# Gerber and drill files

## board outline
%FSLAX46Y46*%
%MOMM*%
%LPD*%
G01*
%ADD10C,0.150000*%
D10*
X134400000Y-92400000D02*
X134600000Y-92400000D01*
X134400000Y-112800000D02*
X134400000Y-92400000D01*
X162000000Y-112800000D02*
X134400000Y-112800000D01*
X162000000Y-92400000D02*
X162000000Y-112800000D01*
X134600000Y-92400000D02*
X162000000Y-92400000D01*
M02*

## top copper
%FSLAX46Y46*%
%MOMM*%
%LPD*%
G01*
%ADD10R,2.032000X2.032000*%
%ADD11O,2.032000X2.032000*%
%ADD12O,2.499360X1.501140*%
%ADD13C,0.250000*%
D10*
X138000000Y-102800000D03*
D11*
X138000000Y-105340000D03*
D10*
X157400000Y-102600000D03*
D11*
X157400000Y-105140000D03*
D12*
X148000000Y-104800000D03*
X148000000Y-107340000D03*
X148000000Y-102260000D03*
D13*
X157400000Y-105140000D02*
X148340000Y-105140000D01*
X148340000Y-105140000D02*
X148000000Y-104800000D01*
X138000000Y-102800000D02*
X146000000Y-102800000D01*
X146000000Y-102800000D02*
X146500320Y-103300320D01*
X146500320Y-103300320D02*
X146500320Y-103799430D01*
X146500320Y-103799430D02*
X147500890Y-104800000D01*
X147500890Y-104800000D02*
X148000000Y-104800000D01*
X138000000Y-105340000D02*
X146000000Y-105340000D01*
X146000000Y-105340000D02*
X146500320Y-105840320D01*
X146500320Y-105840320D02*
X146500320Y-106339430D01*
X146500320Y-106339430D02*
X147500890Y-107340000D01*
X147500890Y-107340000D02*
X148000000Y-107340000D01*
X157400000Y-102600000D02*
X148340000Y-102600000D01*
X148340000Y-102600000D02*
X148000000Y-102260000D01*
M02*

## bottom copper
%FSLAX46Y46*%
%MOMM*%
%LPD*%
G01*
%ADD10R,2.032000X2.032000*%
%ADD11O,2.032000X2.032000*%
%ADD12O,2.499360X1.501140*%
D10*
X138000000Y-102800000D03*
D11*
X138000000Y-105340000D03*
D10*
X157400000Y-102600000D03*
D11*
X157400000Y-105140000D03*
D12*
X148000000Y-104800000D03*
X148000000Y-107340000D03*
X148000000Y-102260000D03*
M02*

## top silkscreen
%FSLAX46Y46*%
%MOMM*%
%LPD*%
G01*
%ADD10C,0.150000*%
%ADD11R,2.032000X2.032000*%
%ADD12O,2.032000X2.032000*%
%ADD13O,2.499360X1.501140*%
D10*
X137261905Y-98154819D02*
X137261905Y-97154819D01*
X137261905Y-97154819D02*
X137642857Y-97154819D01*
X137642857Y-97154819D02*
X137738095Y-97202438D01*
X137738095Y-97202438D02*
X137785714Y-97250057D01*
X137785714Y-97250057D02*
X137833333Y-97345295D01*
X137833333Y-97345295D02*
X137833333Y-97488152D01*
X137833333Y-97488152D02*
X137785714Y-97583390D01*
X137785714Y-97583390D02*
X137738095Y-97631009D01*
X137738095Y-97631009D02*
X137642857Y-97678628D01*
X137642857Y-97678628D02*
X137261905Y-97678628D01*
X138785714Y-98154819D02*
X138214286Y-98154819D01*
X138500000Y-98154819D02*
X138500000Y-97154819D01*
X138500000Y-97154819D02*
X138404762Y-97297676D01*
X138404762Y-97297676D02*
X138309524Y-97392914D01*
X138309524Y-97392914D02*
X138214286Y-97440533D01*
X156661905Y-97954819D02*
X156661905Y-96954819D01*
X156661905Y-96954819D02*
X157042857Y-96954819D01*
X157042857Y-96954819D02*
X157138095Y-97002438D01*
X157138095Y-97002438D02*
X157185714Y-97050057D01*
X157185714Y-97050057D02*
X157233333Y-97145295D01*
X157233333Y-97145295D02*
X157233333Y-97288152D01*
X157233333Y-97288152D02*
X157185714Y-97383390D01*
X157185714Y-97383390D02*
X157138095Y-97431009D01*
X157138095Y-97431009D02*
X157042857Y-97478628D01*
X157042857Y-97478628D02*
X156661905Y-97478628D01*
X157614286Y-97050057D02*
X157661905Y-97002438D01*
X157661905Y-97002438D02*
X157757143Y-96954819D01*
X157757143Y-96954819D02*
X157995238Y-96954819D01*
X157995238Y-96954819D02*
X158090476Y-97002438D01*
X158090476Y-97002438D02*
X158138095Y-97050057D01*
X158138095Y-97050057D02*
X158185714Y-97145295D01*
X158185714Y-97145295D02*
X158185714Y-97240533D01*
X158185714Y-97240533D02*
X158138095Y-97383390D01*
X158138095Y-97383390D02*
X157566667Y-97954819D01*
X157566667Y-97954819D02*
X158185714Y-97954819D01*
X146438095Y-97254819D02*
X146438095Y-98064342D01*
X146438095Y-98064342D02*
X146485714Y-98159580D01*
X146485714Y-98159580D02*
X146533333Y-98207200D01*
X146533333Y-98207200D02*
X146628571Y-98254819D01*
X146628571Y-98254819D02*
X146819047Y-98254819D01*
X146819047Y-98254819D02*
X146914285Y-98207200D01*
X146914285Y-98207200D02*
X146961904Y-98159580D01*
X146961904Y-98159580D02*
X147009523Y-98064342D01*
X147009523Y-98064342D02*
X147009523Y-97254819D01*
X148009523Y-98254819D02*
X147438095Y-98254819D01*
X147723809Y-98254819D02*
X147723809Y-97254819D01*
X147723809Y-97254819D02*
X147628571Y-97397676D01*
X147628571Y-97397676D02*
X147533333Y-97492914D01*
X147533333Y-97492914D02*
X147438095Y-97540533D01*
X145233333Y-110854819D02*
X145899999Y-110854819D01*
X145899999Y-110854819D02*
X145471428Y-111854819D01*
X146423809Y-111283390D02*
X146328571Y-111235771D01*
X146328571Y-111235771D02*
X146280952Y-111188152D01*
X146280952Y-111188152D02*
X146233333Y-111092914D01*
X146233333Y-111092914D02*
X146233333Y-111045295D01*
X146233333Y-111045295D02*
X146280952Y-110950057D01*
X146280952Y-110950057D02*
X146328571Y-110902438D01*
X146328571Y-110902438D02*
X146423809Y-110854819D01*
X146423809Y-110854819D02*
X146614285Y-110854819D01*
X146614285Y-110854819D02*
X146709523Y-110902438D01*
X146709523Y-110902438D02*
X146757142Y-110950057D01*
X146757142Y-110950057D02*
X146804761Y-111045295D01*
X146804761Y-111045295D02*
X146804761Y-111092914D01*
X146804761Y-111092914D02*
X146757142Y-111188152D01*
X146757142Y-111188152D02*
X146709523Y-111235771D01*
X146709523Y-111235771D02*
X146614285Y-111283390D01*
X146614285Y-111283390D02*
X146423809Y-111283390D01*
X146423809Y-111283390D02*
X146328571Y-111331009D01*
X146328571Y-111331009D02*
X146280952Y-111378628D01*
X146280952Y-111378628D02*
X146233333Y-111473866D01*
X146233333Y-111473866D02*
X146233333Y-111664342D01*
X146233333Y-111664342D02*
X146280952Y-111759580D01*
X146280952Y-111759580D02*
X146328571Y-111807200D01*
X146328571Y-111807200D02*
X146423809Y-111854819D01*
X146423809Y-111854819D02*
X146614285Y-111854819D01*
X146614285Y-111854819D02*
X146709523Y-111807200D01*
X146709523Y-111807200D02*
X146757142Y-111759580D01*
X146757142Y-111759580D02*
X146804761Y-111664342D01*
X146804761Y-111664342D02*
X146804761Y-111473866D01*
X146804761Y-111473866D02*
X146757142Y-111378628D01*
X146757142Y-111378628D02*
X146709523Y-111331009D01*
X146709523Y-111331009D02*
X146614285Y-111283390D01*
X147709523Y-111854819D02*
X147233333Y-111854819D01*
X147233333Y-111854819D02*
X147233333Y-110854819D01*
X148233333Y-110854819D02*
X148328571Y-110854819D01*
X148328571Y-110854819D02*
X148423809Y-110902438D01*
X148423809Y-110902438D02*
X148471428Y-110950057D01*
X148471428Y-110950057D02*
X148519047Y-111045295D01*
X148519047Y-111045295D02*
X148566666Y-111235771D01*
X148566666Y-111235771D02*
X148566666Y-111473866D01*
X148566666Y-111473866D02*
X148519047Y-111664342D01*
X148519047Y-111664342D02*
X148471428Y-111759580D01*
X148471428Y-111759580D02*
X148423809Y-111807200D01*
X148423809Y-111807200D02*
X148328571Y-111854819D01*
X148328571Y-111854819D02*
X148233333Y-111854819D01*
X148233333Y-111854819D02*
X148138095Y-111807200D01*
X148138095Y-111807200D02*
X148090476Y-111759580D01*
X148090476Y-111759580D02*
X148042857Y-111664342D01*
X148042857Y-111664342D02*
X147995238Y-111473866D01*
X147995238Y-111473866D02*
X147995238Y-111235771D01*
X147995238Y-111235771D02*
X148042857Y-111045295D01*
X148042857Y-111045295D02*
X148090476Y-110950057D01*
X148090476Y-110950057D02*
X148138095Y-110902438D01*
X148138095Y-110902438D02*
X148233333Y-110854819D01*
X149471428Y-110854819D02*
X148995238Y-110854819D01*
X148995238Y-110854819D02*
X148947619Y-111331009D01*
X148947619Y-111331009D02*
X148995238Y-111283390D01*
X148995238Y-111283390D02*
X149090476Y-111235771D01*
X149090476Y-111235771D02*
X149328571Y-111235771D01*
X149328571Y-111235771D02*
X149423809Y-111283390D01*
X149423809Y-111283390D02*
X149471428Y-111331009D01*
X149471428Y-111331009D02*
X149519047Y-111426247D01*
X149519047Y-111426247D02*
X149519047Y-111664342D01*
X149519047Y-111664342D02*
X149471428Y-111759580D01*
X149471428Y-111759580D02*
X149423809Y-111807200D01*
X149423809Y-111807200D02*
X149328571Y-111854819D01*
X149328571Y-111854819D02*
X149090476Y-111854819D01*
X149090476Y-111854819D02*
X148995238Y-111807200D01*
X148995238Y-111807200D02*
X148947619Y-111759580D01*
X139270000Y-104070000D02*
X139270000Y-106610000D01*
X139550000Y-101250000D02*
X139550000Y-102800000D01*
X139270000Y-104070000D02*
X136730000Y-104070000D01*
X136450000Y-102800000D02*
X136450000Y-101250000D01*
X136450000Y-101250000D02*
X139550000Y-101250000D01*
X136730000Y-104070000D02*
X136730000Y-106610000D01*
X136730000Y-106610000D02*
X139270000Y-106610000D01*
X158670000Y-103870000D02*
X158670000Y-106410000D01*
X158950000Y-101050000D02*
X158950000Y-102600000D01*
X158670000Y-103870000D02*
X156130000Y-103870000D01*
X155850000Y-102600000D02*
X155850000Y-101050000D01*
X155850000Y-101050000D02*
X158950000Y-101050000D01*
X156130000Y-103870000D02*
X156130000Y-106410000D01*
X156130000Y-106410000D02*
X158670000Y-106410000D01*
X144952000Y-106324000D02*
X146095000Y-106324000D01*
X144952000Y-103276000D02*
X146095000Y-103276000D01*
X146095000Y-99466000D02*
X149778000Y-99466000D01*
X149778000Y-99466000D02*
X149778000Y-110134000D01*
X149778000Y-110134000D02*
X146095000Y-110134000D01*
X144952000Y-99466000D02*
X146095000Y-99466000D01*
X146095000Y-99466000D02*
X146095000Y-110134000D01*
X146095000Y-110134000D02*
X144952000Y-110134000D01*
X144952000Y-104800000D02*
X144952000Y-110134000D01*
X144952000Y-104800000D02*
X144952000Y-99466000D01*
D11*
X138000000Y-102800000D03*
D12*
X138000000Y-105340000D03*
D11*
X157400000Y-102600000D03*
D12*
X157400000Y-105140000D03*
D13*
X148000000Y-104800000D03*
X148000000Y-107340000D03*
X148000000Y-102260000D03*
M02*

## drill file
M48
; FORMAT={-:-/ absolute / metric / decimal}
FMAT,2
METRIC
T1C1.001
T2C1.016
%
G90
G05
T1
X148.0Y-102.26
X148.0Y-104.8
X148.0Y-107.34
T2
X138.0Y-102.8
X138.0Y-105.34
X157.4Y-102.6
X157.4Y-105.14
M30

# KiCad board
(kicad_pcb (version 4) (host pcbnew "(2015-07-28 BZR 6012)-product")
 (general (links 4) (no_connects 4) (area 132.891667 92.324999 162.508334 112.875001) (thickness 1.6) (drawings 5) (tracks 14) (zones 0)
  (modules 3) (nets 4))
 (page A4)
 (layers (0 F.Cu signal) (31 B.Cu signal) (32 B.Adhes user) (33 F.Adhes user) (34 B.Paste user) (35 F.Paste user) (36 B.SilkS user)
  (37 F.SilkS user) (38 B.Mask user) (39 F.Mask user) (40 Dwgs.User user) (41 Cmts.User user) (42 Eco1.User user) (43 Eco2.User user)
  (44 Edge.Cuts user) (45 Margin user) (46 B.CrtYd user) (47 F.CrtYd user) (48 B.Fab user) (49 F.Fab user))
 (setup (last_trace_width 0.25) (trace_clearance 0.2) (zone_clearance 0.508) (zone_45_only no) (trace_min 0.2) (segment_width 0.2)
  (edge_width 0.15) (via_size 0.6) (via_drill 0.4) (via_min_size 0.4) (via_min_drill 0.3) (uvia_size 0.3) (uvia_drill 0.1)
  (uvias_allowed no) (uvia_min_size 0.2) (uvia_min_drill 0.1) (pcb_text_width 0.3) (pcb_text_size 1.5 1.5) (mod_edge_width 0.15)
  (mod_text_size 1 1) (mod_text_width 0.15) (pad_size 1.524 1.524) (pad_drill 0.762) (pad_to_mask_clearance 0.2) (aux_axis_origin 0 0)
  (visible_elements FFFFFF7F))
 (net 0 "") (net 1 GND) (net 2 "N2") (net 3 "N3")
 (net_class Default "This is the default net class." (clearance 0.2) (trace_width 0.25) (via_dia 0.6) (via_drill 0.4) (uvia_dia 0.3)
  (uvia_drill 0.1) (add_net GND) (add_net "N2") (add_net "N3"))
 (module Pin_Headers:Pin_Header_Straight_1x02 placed (layer F.Cu) (at 138 102.8)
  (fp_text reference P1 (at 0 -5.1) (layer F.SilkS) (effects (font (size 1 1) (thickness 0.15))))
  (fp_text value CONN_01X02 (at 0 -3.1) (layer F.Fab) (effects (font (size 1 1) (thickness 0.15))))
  (fp_line (start 1.27 1.27) (end 1.27 3.81) (layer F.SilkS) (width 0.15))
  (fp_line (start 1.55 -1.55) (end 1.55 0) (layer F.SilkS) (width 0.15))
  (fp_line (start 1.27 1.27) (end -1.27 1.27) (layer F.SilkS) (width 0.15))
  (fp_line (start -1.55 0) (end -1.55 -1.55) (layer F.SilkS) (width 0.15))
  (fp_line (start -1.55 -1.55) (end 1.55 -1.55) (layer F.SilkS) (width 0.15))
  (fp_line (start -1.27 1.27) (end -1.27 3.81) (layer F.SilkS) (width 0.15))
  (fp_line (start -1.27 3.81) (end 1.27 3.81) (layer F.SilkS) (width 0.15))
  (pad 1 thru_hole rect (at 0 0) (size 2.032 2.032) (drill 1.016) (layers *.Cu *.Mask F.SilkS) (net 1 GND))
  (pad 2 thru_hole oval (at 0 2.54) (size 2.032 2.032) (drill 1.016) (layers *.Cu *.Mask F.SilkS) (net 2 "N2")))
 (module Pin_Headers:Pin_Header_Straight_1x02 (layer F.Cu) (at 157.4 102.6)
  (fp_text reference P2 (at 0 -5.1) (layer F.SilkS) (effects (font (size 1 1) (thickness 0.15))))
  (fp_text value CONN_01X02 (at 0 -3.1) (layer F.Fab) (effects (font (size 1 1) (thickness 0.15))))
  (fp_line (start 1.27 1.27) (end 1.27 3.81) (layer F.SilkS) (width 0.15))
  (fp_line (start 1.55 -1.55) (end 1.55 0) (layer F.SilkS) (width 0.15))
  (fp_line (start 1.27 1.27) (end -1.27 1.27) (layer F.SilkS) (width 0.15))
  (fp_line (start -1.55 0) (end -1.55 -1.55) (layer F.SilkS) (width 0.15))
  (fp_line (start -1.55 -1.55) (end 1.55 -1.55) (layer F.SilkS) (width 0.15))
  (fp_line (start -1.27 1.27) (end -1.27 3.81) (layer F.SilkS) (width 0.15))
  (fp_line (start -1.27 3.81) (end 1.27 3.81) (layer F.SilkS) (width 0.15))
  (pad 1 thru_hole rect (at 0 0) (size 2.032 2.032) (drill 1.016) (layers *.Cu *.Mask F.SilkS) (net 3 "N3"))
  (pad 2 thru_hole oval (at 0 2.54) (size 2.032 2.032) (drill 1.016) (layers *.Cu *.Mask F.SilkS) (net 1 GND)))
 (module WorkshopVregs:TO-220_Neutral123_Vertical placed (layer F.Cu) (at 148 104.8 90)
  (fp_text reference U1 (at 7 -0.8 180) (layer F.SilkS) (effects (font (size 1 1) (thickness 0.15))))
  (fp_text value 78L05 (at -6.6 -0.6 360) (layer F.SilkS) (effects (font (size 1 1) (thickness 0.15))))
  (fp_line (start -1.524 -3.048) (end -1.524 -1.905) (layer F.SilkS) (width 0.15))
  (fp_line (start 1.524 -3.048) (end 1.524 -1.905) (layer F.SilkS) (width 0.15))
  (fp_line (start 5.334 -1.905) (end 5.334 1.778) (layer F.SilkS) (width 0.15))
  (fp_line (start 5.334 1.778) (end -5.334 1.778) (layer F.SilkS) (width 0.15))
  (fp_line (start -5.334 1.778) (end -5.334 -1.905) (layer F.SilkS) (width 0.15))
  (fp_line (start 5.334 -3.048) (end 5.334 -1.905) (layer F.SilkS) (width 0.15))
  (fp_line (start 5.334 -1.905) (end -5.334 -1.905) (layer F.SilkS) (width 0.15))
  (fp_line (start -5.334 -1.905) (end -5.334 -3.048) (layer F.SilkS) (width 0.15))
  (fp_line (start 0 -3.048) (end -5.334 -3.048) (layer F.SilkS) (width 0.15))
  (fp_line (start 0 -3.048) (end 5.334 -3.048) (layer F.SilkS) (width 0.15))
  (pad GND thru_hole oval (at 0 0 180) (size 2.49936 1.50114) (drill 1.00076) (layers *.Cu *.Mask F.SilkS) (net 1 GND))
  (pad VI thru_hole oval (at -2.54 0 180) (size 2.49936 1.50114) (drill 1.00076) (layers *.Cu *.Mask F.SilkS) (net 2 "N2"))
  (pad VO thru_hole oval (at 2.54 0 180) (size 2.49936 1.50114) (drill 1.00076) (layers *.Cu *.Mask F.SilkS) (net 3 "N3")))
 (gr_line (start 134.4 92.4) (end 134.6 92.4) (angle 90) (layer Edge.Cuts) (width 0.15))
 (gr_line (start 134.4 112.8) (end 134.4 92.4) (angle 90) (layer Edge.Cuts) (width 0.15))
 (gr_line (start 162 112.8) (end 134.4 112.8) (angle 90) (layer Edge.Cuts) (width 0.15))
 (gr_line (start 162 92.4) (end 162 112.8) (angle 90) (layer Edge.Cuts) (width 0.15))
 (gr_line (start 134.6 92.4) (end 162 92.4) (angle 90) (layer Edge.Cuts) (width 0.15))
 (segment (start 157.4 105.14) (end 148.34 105.14) (width 0.25) (layer F.Cu) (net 1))
 (segment (start 148.34 105.14) (end 148 104.8) (width 0.25) (layer F.Cu) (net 1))
 (segment (start 138 102.8) (end 146 102.8) (width 0.25) (layer F.Cu) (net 1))
 (segment (start 146 102.8) (end 146.50032 103.30032) (width 0.25) (layer F.Cu) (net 1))
 (segment (start 146.50032 103.30032) (end 146.50032 103.79943) (width 0.25) (layer F.Cu) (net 1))
 (segment (start 146.50032 103.79943) (end 147.50089 104.8) (width 0.25) (layer F.Cu) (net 1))
 (segment (start 147.50089 104.8) (end 148 104.8) (width 0.25) (layer F.Cu) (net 1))
 (segment (start 138 105.34) (end 146 105.34) (width 0.25) (layer F.Cu) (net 2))
 (segment (start 146 105.34) (end 146.50032 105.84032) (width 0.25) (layer F.Cu) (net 2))
 (segment (start 146.50032 105.84032) (end 146.50032 106.33943) (width 0.25) (layer F.Cu) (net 2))
 (segment (start 146.50032 106.33943) (end 147.50089 107.34) (width 0.25) (layer F.Cu) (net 2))
 (segment (start 147.50089 107.34) (end 148 107.34) (width 0.25) (layer F.Cu) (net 2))
 (segment (start 157.4 102.6) (end 148.34 102.6) (width 0.25) (layer F.Cu) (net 3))
 (segment (start 148.34 102.6) (end 148 102.26) (width 0.25) (layer F.Cu) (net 3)))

